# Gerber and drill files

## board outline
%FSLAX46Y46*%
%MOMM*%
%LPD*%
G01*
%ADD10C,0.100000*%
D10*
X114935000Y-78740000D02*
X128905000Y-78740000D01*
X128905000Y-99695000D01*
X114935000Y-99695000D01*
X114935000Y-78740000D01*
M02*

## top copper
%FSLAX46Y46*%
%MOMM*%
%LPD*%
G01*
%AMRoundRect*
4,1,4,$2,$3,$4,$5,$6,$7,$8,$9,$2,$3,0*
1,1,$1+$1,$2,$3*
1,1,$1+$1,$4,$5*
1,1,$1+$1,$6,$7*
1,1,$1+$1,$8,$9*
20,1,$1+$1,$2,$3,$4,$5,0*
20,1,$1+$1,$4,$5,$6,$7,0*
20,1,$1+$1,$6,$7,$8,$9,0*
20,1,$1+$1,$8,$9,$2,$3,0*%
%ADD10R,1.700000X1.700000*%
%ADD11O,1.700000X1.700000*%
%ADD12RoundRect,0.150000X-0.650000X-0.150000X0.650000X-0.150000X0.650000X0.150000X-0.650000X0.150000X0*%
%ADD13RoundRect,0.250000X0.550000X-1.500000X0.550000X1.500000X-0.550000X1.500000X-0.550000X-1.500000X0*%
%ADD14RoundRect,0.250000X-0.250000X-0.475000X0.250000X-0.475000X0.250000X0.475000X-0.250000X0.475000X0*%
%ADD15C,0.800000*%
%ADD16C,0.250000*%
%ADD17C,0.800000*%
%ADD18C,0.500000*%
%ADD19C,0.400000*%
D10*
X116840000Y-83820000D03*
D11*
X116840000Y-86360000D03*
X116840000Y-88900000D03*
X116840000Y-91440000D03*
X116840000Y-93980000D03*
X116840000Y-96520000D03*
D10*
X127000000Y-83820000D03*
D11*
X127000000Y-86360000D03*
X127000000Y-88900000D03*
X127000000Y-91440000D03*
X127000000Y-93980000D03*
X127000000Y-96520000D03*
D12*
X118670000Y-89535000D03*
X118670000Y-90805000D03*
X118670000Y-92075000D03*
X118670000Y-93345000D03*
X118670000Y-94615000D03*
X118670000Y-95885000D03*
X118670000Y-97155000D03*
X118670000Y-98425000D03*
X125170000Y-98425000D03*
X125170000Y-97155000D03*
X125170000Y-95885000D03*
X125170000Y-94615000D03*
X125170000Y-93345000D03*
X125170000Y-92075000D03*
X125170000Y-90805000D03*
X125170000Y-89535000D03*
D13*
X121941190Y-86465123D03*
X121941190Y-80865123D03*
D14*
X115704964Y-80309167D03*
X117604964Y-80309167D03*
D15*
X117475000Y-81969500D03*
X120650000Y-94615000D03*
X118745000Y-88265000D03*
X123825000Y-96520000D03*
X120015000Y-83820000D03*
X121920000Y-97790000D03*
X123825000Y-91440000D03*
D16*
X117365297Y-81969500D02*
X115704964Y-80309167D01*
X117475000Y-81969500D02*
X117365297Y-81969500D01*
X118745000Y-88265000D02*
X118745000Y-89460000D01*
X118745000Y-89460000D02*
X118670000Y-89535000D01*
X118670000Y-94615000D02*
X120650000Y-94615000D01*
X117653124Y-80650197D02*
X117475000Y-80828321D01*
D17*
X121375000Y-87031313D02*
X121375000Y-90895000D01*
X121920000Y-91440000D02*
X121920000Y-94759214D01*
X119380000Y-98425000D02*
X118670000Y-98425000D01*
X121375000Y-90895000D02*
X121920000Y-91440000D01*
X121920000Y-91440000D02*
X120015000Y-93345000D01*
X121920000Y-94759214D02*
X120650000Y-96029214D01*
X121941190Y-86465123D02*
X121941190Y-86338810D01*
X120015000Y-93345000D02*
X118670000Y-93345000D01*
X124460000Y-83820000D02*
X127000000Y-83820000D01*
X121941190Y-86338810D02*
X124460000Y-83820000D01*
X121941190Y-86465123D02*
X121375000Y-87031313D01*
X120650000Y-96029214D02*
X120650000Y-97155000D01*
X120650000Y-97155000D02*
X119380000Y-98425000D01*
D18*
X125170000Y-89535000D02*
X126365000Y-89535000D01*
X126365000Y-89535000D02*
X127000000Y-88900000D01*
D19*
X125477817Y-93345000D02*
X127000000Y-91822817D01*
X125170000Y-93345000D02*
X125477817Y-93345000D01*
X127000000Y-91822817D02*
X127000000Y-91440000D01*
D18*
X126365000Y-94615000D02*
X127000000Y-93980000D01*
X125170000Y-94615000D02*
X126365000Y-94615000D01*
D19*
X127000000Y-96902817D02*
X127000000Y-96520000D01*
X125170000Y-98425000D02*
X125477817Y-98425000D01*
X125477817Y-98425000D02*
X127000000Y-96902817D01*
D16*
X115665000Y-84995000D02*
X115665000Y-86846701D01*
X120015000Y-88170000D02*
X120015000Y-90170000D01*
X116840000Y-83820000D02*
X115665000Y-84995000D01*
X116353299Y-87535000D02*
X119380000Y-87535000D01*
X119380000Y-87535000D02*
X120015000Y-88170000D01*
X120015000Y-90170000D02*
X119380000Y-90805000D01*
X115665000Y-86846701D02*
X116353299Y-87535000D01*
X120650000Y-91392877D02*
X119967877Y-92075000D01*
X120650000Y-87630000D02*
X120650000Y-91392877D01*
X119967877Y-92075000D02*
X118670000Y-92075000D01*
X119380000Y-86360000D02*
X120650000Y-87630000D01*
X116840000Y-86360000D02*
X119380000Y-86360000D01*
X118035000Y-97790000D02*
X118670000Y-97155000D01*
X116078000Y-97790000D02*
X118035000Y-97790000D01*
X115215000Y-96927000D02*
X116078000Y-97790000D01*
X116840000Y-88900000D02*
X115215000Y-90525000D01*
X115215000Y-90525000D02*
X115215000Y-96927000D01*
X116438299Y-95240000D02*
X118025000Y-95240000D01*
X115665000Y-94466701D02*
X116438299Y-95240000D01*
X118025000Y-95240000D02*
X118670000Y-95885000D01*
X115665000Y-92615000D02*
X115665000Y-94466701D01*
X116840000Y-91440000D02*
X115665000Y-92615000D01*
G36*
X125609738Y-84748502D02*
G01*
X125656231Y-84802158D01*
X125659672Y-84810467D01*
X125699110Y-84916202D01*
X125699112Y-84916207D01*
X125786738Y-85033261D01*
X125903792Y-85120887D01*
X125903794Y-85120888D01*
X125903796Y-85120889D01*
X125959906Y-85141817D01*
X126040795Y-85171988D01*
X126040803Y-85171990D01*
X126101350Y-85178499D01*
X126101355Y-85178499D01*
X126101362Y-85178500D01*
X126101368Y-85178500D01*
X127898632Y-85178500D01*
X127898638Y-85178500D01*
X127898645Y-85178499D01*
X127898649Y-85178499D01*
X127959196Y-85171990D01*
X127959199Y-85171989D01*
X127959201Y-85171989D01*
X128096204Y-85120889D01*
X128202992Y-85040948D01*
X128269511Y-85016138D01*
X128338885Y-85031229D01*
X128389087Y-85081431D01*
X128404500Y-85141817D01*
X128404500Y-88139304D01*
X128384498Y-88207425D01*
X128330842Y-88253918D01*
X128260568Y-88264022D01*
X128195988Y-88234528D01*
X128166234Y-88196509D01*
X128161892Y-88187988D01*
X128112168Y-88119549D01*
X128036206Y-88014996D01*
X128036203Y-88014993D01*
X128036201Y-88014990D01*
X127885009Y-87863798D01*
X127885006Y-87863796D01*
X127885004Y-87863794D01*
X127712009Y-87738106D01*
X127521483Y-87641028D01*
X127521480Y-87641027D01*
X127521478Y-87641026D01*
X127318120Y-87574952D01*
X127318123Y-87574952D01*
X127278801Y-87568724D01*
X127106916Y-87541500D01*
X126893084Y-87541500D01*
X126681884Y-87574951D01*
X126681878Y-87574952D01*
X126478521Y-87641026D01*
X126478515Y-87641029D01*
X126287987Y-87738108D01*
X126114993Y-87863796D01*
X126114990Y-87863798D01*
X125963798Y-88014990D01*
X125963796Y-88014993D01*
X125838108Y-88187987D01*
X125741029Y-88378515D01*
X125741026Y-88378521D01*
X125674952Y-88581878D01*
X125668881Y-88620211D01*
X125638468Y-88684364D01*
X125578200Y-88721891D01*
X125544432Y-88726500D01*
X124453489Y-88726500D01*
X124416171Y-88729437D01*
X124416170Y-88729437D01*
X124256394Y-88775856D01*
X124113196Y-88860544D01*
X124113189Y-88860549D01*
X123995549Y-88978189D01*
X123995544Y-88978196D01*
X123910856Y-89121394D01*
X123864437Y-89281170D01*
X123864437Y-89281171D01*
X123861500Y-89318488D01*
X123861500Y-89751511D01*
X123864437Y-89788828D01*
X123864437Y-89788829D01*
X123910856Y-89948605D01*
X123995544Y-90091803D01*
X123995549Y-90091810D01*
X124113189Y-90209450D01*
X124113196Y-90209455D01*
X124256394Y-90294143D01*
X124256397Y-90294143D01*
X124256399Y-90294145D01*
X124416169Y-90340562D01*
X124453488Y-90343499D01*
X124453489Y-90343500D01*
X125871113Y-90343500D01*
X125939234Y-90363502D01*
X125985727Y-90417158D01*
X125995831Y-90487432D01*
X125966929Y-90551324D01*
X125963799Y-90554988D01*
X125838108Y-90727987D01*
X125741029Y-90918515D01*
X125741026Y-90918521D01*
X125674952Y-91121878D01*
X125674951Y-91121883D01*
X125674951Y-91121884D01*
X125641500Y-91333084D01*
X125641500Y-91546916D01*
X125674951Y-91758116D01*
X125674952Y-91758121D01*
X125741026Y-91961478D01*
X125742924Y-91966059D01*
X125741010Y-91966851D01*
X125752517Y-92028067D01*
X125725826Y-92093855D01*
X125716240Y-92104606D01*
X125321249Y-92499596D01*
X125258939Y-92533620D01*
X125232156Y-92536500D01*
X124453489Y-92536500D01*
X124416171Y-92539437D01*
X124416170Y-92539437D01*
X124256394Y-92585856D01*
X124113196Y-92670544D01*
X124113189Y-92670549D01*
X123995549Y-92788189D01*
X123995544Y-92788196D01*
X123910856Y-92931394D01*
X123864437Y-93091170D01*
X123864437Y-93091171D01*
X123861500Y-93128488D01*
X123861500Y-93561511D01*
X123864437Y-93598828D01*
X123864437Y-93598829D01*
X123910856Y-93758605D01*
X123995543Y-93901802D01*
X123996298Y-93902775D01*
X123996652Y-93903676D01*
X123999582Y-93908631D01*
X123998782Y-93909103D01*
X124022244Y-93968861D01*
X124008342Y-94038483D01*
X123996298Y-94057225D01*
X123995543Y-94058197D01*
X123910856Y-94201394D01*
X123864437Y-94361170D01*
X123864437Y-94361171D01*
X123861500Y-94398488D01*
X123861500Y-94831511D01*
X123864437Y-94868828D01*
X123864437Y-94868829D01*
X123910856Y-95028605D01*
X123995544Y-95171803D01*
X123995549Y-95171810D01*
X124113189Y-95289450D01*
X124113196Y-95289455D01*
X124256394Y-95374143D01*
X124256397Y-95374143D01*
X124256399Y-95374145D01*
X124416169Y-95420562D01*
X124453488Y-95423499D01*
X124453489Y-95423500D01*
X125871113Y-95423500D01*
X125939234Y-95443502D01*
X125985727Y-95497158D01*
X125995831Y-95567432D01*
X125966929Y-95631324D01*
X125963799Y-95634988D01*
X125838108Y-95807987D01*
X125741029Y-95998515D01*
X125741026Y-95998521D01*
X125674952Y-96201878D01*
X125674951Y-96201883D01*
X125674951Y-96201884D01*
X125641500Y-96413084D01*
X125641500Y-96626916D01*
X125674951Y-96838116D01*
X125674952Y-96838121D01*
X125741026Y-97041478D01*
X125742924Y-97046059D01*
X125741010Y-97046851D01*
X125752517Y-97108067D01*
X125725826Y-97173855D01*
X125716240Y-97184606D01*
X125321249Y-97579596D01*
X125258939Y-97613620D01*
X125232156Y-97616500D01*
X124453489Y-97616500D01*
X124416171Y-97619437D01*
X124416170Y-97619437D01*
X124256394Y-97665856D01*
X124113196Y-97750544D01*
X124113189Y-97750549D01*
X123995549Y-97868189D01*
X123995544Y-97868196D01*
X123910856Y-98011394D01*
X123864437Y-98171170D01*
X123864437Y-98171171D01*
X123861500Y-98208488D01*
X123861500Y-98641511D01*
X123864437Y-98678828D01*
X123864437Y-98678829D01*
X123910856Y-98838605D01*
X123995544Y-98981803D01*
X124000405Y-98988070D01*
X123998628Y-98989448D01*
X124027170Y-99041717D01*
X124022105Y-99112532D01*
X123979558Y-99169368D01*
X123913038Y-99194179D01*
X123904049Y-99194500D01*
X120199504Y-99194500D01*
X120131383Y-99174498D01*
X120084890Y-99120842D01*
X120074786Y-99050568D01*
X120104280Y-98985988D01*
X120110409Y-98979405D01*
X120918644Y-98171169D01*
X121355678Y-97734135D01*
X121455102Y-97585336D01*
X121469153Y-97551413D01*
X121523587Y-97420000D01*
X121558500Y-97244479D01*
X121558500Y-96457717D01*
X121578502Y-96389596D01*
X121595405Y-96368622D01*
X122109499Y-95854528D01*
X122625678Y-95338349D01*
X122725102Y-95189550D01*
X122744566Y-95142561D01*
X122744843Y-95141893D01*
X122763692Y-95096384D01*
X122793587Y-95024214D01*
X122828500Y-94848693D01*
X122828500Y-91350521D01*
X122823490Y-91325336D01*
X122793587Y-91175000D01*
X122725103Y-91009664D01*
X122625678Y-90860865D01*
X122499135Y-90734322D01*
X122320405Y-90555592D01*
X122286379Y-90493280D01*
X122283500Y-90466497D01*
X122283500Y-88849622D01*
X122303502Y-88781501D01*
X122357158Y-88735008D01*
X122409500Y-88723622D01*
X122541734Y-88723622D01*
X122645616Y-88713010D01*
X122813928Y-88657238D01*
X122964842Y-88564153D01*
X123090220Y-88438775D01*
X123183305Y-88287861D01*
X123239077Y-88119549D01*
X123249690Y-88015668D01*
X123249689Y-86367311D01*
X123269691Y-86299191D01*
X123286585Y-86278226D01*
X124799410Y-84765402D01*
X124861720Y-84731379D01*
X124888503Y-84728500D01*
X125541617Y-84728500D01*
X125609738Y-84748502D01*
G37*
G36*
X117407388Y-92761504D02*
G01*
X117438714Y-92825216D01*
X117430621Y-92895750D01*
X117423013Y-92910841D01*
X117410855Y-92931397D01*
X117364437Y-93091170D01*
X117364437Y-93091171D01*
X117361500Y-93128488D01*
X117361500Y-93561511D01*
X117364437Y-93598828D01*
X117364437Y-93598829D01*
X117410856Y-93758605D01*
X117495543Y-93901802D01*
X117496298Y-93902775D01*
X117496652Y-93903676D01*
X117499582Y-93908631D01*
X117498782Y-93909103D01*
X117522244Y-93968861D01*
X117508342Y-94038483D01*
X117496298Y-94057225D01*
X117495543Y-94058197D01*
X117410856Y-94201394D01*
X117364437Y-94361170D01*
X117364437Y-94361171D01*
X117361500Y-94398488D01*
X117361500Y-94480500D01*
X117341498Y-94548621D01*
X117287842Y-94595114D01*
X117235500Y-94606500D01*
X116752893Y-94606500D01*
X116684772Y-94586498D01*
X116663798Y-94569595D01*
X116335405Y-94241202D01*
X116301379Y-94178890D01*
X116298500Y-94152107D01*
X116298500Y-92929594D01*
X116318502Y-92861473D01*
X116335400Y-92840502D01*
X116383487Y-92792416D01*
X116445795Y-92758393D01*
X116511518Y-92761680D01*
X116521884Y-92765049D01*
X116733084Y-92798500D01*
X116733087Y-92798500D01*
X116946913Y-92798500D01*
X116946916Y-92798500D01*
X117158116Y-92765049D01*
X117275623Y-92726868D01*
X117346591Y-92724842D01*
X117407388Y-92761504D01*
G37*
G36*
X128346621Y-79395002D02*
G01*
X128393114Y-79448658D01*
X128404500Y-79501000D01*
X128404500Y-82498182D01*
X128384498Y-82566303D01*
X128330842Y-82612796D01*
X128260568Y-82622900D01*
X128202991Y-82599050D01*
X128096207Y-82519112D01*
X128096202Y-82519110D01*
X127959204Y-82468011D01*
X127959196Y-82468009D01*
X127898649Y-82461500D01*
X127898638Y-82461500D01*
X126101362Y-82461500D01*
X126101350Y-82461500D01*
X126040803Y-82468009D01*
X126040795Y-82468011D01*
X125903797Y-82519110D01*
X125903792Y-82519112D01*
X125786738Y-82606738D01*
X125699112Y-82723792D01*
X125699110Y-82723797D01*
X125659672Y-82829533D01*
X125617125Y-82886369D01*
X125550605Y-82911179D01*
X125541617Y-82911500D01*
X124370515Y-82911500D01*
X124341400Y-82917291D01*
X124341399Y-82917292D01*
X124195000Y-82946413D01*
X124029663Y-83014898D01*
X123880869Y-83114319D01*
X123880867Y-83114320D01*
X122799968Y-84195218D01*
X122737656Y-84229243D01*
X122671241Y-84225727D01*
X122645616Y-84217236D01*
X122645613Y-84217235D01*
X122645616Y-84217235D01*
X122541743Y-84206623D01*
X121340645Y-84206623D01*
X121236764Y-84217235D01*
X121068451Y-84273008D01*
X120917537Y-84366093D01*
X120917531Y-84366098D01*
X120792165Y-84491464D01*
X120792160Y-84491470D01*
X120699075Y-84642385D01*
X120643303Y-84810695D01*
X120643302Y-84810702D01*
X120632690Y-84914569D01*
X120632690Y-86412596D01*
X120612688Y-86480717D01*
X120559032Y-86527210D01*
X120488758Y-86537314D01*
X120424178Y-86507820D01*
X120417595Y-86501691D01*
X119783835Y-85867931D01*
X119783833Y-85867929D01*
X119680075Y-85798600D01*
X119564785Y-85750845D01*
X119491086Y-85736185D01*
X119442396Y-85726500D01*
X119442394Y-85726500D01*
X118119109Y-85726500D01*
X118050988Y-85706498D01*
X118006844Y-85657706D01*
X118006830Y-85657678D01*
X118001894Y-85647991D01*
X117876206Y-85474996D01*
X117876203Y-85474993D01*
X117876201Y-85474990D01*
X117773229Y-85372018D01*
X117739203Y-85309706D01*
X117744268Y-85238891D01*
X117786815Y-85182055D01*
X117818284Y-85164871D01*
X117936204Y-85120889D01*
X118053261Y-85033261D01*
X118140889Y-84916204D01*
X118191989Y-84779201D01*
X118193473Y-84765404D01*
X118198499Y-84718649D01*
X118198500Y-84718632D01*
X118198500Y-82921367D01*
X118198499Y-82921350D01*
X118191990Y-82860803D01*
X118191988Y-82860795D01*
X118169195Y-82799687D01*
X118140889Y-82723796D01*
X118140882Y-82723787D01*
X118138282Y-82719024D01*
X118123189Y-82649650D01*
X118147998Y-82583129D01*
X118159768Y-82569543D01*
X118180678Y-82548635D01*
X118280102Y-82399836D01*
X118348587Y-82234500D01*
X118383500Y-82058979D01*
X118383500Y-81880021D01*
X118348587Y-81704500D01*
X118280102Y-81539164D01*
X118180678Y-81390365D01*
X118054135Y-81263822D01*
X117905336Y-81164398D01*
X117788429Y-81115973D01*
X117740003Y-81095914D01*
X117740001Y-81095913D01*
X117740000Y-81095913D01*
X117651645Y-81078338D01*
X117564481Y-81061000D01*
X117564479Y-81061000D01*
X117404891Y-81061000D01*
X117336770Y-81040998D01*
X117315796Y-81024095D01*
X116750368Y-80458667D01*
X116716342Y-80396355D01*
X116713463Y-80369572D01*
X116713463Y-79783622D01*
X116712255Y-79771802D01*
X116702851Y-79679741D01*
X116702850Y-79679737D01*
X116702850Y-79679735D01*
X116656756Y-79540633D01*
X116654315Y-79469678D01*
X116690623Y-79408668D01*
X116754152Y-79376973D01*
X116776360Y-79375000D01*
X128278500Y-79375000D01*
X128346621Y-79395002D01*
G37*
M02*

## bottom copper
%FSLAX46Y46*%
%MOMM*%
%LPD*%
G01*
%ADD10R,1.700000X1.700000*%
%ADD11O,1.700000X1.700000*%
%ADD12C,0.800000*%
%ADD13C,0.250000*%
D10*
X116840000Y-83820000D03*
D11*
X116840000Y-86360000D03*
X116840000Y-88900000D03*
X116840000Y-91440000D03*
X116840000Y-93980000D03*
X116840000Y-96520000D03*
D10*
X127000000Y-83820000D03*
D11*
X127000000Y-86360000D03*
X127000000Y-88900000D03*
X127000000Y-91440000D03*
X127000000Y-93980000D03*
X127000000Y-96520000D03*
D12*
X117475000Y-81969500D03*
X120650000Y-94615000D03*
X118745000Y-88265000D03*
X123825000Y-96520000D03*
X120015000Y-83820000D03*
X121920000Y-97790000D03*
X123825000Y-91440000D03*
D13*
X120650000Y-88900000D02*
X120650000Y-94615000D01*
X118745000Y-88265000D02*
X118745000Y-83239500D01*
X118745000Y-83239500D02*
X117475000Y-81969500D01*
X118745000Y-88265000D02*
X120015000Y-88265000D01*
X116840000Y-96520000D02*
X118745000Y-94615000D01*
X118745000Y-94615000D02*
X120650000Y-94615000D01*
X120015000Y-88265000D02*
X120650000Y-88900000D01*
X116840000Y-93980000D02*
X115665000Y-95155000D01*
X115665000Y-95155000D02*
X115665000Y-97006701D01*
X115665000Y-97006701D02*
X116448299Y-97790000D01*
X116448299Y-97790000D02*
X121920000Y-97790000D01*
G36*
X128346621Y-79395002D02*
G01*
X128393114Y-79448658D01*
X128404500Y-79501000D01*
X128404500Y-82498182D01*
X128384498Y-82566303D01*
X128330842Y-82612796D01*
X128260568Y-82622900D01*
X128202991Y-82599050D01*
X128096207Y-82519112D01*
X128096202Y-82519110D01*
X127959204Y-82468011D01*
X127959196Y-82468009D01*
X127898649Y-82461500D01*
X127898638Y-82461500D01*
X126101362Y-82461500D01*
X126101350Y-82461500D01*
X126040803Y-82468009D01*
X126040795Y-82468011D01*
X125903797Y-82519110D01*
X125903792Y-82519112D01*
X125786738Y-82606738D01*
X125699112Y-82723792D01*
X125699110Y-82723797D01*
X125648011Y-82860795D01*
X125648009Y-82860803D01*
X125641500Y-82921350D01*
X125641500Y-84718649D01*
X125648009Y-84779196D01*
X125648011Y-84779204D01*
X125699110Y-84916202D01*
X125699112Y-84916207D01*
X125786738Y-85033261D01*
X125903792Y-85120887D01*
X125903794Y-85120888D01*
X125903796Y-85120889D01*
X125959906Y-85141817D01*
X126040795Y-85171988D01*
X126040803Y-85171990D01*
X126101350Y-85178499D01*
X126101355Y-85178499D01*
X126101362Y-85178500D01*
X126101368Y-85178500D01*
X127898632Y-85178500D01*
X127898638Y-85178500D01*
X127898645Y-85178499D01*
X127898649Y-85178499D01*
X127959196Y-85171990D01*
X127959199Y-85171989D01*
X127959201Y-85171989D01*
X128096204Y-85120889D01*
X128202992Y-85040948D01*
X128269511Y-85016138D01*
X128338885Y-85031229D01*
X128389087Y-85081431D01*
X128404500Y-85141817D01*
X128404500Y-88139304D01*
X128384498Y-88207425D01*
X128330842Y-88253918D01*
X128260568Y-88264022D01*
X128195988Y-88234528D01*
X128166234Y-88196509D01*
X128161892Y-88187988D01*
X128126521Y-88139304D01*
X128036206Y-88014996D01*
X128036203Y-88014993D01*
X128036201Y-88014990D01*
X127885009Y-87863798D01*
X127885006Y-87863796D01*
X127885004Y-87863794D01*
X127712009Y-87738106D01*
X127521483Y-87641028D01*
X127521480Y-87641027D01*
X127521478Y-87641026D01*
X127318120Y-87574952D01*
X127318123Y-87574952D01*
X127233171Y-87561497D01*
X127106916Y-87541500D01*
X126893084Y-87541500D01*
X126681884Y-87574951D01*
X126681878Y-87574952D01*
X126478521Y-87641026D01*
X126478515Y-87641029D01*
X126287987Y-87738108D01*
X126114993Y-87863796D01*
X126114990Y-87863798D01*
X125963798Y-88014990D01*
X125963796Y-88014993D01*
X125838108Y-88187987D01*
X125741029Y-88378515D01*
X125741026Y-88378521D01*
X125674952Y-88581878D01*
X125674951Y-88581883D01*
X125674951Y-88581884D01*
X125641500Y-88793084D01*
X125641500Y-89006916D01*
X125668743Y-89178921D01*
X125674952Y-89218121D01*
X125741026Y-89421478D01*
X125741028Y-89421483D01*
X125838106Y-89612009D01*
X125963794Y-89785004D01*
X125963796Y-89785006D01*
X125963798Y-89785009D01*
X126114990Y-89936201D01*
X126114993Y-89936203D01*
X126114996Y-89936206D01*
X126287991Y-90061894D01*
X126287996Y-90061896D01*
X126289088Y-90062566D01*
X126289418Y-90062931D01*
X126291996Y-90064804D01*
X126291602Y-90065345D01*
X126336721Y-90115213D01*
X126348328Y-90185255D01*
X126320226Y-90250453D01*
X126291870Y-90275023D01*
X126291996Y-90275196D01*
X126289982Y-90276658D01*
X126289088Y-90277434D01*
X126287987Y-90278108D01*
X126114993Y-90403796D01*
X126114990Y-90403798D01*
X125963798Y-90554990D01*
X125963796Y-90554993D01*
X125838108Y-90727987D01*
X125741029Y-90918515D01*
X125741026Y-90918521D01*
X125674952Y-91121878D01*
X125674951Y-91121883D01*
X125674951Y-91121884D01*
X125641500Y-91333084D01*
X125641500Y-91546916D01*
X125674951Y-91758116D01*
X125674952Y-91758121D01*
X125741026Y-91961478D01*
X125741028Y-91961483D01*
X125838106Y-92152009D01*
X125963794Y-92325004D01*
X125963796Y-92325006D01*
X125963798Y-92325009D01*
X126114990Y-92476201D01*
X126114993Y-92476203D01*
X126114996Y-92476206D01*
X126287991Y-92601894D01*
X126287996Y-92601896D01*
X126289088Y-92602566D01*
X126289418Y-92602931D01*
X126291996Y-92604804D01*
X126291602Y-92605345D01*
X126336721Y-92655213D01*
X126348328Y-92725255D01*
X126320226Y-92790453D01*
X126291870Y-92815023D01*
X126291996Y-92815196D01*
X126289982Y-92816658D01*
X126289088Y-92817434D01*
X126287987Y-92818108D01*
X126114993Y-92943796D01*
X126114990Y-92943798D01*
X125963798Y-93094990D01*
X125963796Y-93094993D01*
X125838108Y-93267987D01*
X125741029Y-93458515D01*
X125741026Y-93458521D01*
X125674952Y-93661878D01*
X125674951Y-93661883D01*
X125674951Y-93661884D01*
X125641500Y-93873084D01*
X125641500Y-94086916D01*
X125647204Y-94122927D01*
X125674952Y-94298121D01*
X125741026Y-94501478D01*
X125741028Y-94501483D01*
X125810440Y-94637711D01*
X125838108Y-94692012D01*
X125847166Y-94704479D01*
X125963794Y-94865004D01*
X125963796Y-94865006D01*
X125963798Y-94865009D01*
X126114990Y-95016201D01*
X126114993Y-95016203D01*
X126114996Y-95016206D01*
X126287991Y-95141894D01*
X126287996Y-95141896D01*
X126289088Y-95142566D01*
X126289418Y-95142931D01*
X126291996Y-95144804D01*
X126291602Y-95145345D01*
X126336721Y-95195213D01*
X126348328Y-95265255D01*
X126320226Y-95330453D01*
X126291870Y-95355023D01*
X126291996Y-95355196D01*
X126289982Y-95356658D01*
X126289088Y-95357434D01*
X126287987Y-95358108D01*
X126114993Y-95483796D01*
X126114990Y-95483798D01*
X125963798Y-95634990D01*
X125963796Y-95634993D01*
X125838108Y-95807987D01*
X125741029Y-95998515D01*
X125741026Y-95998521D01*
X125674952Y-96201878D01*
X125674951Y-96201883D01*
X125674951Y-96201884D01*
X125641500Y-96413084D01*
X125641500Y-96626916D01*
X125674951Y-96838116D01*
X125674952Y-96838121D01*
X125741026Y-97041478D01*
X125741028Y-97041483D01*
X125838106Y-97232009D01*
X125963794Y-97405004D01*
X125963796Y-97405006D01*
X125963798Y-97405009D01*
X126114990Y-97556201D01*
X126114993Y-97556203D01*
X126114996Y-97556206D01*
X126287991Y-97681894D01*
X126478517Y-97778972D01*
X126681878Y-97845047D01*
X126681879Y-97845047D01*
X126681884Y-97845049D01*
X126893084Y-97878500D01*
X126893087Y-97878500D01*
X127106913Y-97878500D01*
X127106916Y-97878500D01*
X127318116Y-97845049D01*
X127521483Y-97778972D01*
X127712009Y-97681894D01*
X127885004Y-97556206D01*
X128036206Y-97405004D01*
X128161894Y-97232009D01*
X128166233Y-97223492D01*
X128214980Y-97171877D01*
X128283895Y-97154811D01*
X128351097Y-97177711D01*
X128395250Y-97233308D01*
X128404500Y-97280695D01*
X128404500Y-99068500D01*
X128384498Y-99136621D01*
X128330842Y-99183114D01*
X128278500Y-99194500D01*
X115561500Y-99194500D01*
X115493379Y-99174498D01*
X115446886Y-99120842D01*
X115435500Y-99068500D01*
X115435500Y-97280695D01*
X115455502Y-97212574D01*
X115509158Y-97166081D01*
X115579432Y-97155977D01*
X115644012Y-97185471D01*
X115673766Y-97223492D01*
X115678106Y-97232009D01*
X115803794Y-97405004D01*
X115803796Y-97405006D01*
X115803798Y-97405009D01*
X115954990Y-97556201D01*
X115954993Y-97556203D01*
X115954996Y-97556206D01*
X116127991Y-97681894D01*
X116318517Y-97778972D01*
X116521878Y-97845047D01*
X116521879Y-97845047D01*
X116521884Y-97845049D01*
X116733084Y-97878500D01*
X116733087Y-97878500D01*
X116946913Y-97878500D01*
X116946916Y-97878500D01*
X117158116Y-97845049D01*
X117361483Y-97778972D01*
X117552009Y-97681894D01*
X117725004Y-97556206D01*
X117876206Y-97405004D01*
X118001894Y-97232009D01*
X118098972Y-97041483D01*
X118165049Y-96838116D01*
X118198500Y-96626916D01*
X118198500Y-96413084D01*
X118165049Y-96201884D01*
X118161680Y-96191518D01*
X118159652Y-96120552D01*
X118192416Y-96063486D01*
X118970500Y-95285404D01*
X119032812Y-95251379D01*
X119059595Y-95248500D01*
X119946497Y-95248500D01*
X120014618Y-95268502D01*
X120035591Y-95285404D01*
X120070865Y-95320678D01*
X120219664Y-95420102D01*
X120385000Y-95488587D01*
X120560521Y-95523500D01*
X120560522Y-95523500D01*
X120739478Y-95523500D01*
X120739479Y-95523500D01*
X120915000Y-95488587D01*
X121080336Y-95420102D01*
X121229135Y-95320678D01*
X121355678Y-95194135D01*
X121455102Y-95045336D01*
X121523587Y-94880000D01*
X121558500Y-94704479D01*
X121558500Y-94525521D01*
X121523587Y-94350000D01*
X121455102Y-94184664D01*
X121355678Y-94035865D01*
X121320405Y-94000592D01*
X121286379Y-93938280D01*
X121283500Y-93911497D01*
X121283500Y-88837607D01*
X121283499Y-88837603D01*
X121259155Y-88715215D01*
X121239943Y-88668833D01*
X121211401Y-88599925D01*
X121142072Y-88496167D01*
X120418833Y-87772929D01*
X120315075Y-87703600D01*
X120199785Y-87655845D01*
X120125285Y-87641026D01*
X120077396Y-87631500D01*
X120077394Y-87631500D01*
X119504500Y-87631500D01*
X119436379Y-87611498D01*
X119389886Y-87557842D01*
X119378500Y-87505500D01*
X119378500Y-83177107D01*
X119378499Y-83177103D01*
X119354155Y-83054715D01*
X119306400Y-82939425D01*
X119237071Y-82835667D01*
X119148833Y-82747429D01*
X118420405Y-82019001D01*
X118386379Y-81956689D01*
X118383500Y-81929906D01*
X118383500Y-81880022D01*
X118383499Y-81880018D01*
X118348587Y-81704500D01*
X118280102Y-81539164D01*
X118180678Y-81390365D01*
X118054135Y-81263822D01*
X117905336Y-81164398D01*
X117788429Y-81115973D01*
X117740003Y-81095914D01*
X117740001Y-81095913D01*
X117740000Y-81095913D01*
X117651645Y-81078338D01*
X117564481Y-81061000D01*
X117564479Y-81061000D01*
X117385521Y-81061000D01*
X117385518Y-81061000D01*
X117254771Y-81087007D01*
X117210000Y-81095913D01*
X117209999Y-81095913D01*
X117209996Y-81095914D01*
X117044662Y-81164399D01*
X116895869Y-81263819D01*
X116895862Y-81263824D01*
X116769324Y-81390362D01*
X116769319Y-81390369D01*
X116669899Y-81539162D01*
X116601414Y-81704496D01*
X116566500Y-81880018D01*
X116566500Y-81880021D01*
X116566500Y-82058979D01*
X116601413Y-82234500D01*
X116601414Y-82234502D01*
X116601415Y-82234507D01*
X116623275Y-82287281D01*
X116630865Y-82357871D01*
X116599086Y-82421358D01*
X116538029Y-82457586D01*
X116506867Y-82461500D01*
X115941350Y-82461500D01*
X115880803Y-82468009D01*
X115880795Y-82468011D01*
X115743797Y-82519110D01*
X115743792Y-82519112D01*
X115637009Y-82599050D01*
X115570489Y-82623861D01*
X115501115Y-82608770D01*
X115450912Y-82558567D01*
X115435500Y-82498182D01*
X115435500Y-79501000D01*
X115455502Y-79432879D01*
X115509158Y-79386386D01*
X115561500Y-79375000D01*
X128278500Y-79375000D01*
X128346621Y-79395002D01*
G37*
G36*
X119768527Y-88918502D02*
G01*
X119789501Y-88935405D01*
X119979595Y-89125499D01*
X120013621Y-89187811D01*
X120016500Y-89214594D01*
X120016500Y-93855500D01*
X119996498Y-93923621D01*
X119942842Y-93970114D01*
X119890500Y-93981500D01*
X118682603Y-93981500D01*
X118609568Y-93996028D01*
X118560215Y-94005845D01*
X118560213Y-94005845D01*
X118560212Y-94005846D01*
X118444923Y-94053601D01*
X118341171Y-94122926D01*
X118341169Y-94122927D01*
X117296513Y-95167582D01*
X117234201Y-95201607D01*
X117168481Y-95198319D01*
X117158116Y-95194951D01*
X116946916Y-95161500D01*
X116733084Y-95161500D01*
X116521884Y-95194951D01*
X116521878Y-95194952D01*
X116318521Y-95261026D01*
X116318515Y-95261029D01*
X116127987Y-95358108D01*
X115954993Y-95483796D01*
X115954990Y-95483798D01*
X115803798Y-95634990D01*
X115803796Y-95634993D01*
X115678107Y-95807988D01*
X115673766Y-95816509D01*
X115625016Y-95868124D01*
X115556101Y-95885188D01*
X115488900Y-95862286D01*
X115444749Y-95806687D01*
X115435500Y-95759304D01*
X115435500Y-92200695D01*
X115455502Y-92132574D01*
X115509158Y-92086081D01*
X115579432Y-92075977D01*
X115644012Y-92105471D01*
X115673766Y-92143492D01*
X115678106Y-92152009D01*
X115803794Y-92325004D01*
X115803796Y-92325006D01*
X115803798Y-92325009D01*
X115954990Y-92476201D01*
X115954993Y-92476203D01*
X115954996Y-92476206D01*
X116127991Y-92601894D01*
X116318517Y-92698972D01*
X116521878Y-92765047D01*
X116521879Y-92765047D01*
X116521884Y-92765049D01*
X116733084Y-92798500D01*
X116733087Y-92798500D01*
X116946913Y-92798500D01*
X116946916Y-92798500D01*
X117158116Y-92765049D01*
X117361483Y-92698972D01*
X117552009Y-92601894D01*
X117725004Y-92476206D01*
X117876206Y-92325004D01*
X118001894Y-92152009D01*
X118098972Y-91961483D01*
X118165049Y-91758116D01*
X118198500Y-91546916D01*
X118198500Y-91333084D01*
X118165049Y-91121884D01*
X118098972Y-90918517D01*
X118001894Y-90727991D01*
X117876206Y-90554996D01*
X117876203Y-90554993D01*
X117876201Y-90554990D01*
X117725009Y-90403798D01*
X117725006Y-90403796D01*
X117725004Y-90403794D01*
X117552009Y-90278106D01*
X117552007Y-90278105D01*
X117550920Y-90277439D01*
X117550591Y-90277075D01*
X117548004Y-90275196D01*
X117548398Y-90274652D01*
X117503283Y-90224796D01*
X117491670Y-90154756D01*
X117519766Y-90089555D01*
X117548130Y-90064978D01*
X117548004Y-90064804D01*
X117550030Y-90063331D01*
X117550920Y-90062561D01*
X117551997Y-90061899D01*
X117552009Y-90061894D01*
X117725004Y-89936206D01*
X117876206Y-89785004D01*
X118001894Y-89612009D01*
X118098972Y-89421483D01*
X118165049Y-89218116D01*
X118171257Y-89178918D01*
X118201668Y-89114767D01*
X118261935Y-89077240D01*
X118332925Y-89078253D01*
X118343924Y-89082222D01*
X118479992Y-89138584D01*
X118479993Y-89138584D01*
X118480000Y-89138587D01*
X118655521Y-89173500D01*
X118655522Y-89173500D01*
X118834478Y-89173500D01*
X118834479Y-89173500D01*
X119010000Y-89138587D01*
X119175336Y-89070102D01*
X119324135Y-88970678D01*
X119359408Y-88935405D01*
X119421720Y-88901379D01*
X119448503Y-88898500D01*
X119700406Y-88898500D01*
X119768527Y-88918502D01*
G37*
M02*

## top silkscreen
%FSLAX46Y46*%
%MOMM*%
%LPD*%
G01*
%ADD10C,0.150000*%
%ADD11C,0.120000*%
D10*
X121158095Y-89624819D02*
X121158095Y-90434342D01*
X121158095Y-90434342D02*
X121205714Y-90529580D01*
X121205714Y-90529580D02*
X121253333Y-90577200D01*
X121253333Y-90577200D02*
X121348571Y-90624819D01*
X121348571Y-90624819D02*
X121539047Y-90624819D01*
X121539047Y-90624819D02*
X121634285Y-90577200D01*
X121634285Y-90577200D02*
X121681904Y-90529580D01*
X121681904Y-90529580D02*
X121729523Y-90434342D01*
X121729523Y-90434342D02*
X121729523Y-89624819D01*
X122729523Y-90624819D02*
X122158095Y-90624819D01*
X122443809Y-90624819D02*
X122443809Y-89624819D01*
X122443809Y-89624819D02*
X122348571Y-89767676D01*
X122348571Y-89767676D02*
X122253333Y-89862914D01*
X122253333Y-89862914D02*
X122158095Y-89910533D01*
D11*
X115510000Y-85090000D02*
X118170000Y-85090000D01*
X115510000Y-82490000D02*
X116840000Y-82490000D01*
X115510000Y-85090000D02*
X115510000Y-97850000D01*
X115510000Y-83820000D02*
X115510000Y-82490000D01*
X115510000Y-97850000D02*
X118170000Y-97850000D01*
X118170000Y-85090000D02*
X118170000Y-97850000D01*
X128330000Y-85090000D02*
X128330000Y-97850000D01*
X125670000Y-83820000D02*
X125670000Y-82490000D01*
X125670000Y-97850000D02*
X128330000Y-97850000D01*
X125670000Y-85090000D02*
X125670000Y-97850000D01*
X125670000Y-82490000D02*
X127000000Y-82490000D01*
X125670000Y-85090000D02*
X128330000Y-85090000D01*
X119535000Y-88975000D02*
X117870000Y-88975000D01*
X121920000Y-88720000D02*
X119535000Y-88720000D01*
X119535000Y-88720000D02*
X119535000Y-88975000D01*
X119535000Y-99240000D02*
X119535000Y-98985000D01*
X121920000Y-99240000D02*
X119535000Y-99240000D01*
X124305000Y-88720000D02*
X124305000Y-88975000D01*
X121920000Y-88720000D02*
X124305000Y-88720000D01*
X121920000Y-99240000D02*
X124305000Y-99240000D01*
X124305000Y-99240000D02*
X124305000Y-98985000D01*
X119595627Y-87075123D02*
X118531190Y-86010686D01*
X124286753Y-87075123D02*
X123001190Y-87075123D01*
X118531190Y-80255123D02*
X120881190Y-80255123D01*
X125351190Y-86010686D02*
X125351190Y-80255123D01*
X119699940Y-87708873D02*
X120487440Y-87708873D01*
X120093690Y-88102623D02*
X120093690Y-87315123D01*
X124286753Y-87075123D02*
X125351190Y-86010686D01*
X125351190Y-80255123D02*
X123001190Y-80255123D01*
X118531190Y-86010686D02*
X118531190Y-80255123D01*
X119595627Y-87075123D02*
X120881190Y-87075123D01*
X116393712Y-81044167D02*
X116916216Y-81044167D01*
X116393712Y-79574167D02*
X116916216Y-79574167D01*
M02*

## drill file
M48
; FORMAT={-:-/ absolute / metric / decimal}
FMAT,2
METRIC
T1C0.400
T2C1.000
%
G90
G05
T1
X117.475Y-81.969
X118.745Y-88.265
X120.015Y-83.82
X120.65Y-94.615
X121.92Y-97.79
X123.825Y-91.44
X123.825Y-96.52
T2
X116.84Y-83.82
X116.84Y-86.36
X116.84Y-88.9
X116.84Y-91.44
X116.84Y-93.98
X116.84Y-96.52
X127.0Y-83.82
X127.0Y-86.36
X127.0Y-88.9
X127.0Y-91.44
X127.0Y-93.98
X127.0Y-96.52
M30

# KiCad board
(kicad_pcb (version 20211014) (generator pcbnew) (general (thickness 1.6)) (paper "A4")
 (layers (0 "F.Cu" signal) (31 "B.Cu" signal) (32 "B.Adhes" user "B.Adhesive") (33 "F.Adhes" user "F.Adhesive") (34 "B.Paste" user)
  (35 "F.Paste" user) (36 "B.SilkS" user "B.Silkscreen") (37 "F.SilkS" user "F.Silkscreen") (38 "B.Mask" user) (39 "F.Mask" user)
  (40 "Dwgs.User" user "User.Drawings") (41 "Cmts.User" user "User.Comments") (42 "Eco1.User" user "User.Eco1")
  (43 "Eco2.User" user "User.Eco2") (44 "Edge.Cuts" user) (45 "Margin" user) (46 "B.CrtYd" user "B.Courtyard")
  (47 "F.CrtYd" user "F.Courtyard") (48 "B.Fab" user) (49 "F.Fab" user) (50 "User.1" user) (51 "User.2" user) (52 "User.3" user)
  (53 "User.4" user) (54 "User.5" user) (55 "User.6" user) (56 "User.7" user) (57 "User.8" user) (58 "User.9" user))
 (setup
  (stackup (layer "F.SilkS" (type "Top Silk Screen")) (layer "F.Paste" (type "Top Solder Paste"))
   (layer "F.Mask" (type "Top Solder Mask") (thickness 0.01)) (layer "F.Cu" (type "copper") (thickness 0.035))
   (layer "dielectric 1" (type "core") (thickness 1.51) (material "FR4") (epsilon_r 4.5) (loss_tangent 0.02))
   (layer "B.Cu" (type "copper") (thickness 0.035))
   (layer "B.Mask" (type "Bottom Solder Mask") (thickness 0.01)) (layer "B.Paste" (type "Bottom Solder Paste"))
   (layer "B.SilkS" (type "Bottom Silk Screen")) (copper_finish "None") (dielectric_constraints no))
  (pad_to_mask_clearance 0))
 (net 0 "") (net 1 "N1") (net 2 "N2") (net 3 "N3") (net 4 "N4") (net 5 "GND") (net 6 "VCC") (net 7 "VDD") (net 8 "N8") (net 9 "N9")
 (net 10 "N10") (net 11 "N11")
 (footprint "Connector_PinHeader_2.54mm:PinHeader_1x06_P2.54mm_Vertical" (layer "F.Cu") (at 116.84 83.82)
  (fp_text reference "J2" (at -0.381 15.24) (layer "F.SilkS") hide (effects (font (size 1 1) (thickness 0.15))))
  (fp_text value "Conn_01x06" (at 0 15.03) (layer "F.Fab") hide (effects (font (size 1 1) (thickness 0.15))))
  (fp_line (start -1.33 1.27) (end 1.33 1.27) (layer "F.SilkS") (width 0.12))
  (fp_line (start -1.33 -1.33) (end 0 -1.33) (layer "F.SilkS") (width 0.12))
  (fp_line (start -1.33 1.27) (end -1.33 14.03) (layer "F.SilkS") (width 0.12))
  (fp_line (start -1.33 0) (end -1.33 -1.33) (layer "F.SilkS") (width 0.12))
  (fp_line (start -1.33 14.03) (end 1.33 14.03) (layer "F.SilkS") (width 0.12))
  (fp_line (start 1.33 1.27) (end 1.33 14.03) (layer "F.SilkS") (width 0.12))
  (pad "1" thru_hole rect (at 0 0) (size 1.7 1.7) (drill 1) (layers *.Cu *.Mask) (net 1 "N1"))
  (pad "2" thru_hole oval (at 0 2.54) (size 1.7 1.7) (drill 1) (layers *.Cu *.Mask) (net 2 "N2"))
  (pad "3" thru_hole oval (at 0 5.08) (size 1.7 1.7) (drill 1) (layers *.Cu *.Mask) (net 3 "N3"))
  (pad "4" thru_hole oval (at 0 7.62) (size 1.7 1.7) (drill 1) (layers *.Cu *.Mask) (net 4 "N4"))
  (pad "5" thru_hole oval (at 0 10.16) (size 1.7 1.7) (drill 1) (layers *.Cu *.Mask) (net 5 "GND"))
  (pad "6" thru_hole oval (at 0 12.7) (size 1.7 1.7) (drill 1) (layers *.Cu *.Mask) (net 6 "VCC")))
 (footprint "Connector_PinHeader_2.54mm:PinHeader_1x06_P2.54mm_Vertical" (layer "F.Cu") (at 127 83.82)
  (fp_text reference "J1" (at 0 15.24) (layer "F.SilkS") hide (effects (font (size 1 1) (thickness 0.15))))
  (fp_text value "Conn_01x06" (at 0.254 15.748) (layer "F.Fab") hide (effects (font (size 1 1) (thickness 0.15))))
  (fp_line (start 1.33 1.27) (end 1.33 14.03) (layer "F.SilkS") (width 0.12))
  (fp_line (start -1.33 0) (end -1.33 -1.33) (layer "F.SilkS") (width 0.12))
  (fp_line (start -1.33 14.03) (end 1.33 14.03) (layer "F.SilkS") (width 0.12))
  (fp_line (start -1.33 1.27) (end -1.33 14.03) (layer "F.SilkS") (width 0.12))
  (fp_line (start -1.33 -1.33) (end 0 -1.33) (layer "F.SilkS") (width 0.12))
  (fp_line (start -1.33 1.27) (end 1.33 1.27) (layer "F.SilkS") (width 0.12))
  (pad "1" thru_hole rect (at 0 0) (size 1.7 1.7) (drill 1) (layers *.Cu *.Mask) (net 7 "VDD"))
  (pad "2" thru_hole oval (at 0 2.54) (size 1.7 1.7) (drill 1) (layers *.Cu *.Mask) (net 5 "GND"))
  (pad "3" thru_hole oval (at 0 5.08) (size 1.7 1.7) (drill 1) (layers *.Cu *.Mask) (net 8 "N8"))
  (pad "4" thru_hole oval (at 0 7.62) (size 1.7 1.7) (drill 1) (layers *.Cu *.Mask) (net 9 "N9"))
  (pad "5" thru_hole oval (at 0 10.16) (size 1.7 1.7) (drill 1) (layers *.Cu *.Mask) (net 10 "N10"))
  (pad "6" thru_hole oval (at 0 12.7) (size 1.7 1.7) (drill 1) (layers *.Cu *.Mask) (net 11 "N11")))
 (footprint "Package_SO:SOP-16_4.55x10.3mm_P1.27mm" (layer "F.Cu") (at 121.92 93.98)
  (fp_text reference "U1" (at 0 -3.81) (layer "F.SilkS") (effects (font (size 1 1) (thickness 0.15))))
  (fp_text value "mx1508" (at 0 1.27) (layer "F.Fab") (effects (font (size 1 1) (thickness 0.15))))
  (fp_line (start -2.385 -5.005) (end -4.05 -5.005) (layer "F.SilkS") (width 0.12))
  (fp_line (start 0 -5.26) (end -2.385 -5.26) (layer "F.SilkS") (width 0.12))
  (fp_line (start -2.385 -5.26) (end -2.385 -5.005) (layer "F.SilkS") (width 0.12))
  (fp_line (start -2.385 5.26) (end -2.385 5.005) (layer "F.SilkS") (width 0.12))
  (fp_line (start 0 5.26) (end -2.385 5.26) (layer "F.SilkS") (width 0.12))
  (fp_line (start 2.385 -5.26) (end 2.385 -5.005) (layer "F.SilkS") (width 0.12))
  (fp_line (start 0 -5.26) (end 2.385 -5.26) (layer "F.SilkS") (width 0.12))
  (fp_line (start 0 5.26) (end 2.385 5.26) (layer "F.SilkS") (width 0.12))
  (fp_line (start 2.385 5.26) (end 2.385 5.005) (layer "F.SilkS") (width 0.12))
  (pad "1" smd roundrect (at -3.25 -4.445) (size 1.6 0.6) (layers "F.Cu" "F.Paste" "F.Mask") (roundrect_rratio 0.25) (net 6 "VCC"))
  (pad "2" smd roundrect (at -3.25 -3.175) (size 1.6 0.6) (layers "F.Cu" "F.Paste" "F.Mask") (roundrect_rratio 0.25) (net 1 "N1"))
  (pad "3" smd roundrect (at -3.25 -1.905) (size 1.6 0.6) (layers "F.Cu" "F.Paste" "F.Mask") (roundrect_rratio 0.25) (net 2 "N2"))
  (pad "4" smd roundrect (at -3.25 -0.635) (size 1.6 0.6) (layers "F.Cu" "F.Paste" "F.Mask") (roundrect_rratio 0.25) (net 7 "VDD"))
  (pad "5" smd roundrect (at -3.25 0.635) (size 1.6 0.6) (layers "F.Cu" "F.Paste" "F.Mask") (roundrect_rratio 0.25) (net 6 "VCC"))
  (pad "6" smd roundrect (at -3.25 1.905) (size 1.6 0.6) (layers "F.Cu" "F.Paste" "F.Mask") (roundrect_rratio 0.25) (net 4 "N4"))
  (pad "7" smd roundrect (at -3.25 3.175) (size 1.6 0.6) (layers "F.Cu" "F.Paste" "F.Mask") (roundrect_rratio 0.25) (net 3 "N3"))
  (pad "8" smd roundrect (at -3.25 4.445) (size 1.6 0.6) (layers "F.Cu" "F.Paste" "F.Mask") (roundrect_rratio 0.25) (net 7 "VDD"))
  (pad "9" smd roundrect (at 3.25 4.445) (size 1.6 0.6) (layers "F.Cu" "F.Paste" "F.Mask") (roundrect_rratio 0.25) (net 11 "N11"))
  (pad "10" smd roundrect (at 3.25 3.175) (size 1.6 0.6) (layers "F.Cu" "F.Paste" "F.Mask") (roundrect_rratio 0.25) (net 5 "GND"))
  (pad "11" smd roundrect (at 3.25 1.905) (size 1.6 0.6) (layers "F.Cu" "F.Paste" "F.Mask") (roundrect_rratio 0.25) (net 5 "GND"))
  (pad "12" smd roundrect (at 3.25 0.635) (size 1.6 0.6) (layers "F.Cu" "F.Paste" "F.Mask") (roundrect_rratio 0.25) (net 10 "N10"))
  (pad "13" smd roundrect (at 3.25 -0.635) (size 1.6 0.6) (layers "F.Cu" "F.Paste" "F.Mask") (roundrect_rratio 0.25) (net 9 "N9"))
  (pad "14" smd roundrect (at 3.25 -1.905) (size 1.6 0.6) (layers "F.Cu" "F.Paste" "F.Mask") (roundrect_rratio 0.25) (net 5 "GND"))
  (pad "15" smd roundrect (at 3.25 -3.175) (size 1.6 0.6) (layers "F.Cu" "F.Paste" "F.Mask") (roundrect_rratio 0.25) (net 5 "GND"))
  (pad "16" smd roundrect (at 3.25 -4.445) (size 1.6 0.6) (layers "F.Cu" "F.Paste" "F.Mask") (roundrect_rratio 0.25) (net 8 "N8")))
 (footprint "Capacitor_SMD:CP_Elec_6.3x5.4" (layer "F.Cu") (at 121.94119 83.665123 90)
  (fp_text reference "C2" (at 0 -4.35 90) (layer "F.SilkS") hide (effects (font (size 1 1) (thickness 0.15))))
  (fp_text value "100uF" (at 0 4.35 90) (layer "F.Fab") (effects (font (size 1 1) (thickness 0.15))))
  (fp_line (start -3.41 -2.345563) (end -2.345563 -3.41) (layer "F.SilkS") (width 0.12))
  (fp_line (start -3.41 2.345563) (end -3.41 1.06) (layer "F.SilkS") (width 0.12))
  (fp_line (start 3.41 -3.41) (end 3.41 -1.06) (layer "F.SilkS") (width 0.12))
  (fp_line (start -2.345563 3.41) (end 3.41 3.41) (layer "F.SilkS") (width 0.12))
  (fp_line (start -4.04375 -2.24125) (end -4.04375 -1.45375) (layer "F.SilkS") (width 0.12))
  (fp_line (start -4.4375 -1.8475) (end -3.65 -1.8475) (layer "F.SilkS") (width 0.12))
  (fp_line (start -3.41 2.345563) (end -2.345563 3.41) (layer "F.SilkS") (width 0.12))
  (fp_line (start 3.41 3.41) (end 3.41 1.06) (layer "F.SilkS") (width 0.12))
  (fp_line (start -2.345563 -3.41) (end 3.41 -3.41) (layer "F.SilkS") (width 0.12))
  (fp_line (start -3.41 -2.345563) (end -3.41 -1.06) (layer "F.SilkS") (width 0.12))
  (pad "1" smd roundrect (at -2.8 0 90) (size 3.5 1.6) (layers "F.Cu" "F.Paste" "F.Mask") (roundrect_rratio 0.15625) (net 7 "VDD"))
  (pad "2" smd roundrect (at 2.8 0 90) (size 3.5 1.6) (layers "F.Cu" "F.Paste" "F.Mask") (roundrect_rratio 0.15625) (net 5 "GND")))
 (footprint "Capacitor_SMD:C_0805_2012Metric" (layer "F.Cu") (at 116.654964 80.309167)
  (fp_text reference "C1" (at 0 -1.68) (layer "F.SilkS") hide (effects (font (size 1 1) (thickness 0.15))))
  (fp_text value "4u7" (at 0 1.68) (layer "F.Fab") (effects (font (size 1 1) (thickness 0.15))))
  (fp_line (start -0.261252 0.735) (end 0.261252 0.735) (layer "F.SilkS") (width 0.12))
  (fp_line (start -0.261252 -0.735) (end 0.261252 -0.735) (layer "F.SilkS") (width 0.12))
  (pad "1" smd roundrect (at -0.95 0) (size 1 1.45) (layers "F.Cu" "F.Paste" "F.Mask") (roundrect_rratio 0.25) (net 6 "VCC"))
  (pad "2" smd roundrect (at 0.95 0) (size 1 1.45) (layers "F.Cu" "F.Paste" "F.Mask") (roundrect_rratio 0.25) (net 5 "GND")))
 (gr_rect (start 128.905 78.74) (end 114.935 99.695) (layer "Edge.Cuts") (width 0.1) (fill none))
 (segment (start 117.365297 81.9695) (end 115.704964 80.309167) (width 0.25) (layer "F.Cu") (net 6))
 (segment (start 117.475 81.9695) (end 117.365297 81.9695) (width 0.25) (layer "F.Cu") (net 6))
 (segment (start 118.745 88.265) (end 118.745 89.46) (width 0.25) (layer "F.Cu") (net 6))
 (segment (start 118.745 89.46) (end 118.67 89.535) (width 0.25) (layer "F.Cu") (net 6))
 (segment (start 118.67 94.615) (end 120.65 94.615) (width 0.25) (layer "F.Cu") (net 6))
 (via (at 117.475 81.9695) (size 0.8) (drill 0.4) (layers "F.Cu" "B.Cu") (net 6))
 (via (at 120.65 94.615) (size 0.8) (drill 0.4) (layers "F.Cu" "B.Cu") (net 6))
 (via (at 118.745 88.265) (size 0.8) (drill 0.4) (layers "F.Cu" "B.Cu") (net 6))
 (segment (start 120.65 88.9) (end 120.65 94.615) (width 0.25) (layer "B.Cu") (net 6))
 (segment (start 118.745 88.265) (end 118.745 83.2395) (width 0.25) (layer "B.Cu") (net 6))
 (segment (start 118.745 83.2395) (end 117.475 81.9695) (width 0.25) (layer "B.Cu") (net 6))
 (segment (start 118.745 88.265) (end 120.015 88.265) (width 0.25) (layer "B.Cu") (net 6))
 (segment (start 116.84 96.52) (end 118.745 94.615) (width 0.25) (layer "B.Cu") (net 6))
 (segment (start 118.745 94.615) (end 120.65 94.615) (width 0.25) (layer "B.Cu") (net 6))
 (segment (start 120.015 88.265) (end 120.65 88.9) (width 0.25) (layer "B.Cu") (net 6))
 (segment (start 117.653124 80.650197) (end 117.475 80.828321) (width 0.25) (layer "F.Cu") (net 5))
 (via (at 123.825 96.52) (size 0.8) (drill 0.4) (layers "F.Cu" "B.Cu") (free) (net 5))
 (via (at 120.015 83.82) (size 0.8) (drill 0.4) (layers "F.Cu" "B.Cu") (free) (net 5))
 (via (at 121.92 97.79) (size 0.8) (drill 0.4) (layers "F.Cu" "B.Cu") (free) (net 5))
 (via (at 123.825 91.44) (size 0.8) (drill 0.4) (layers "F.Cu" "B.Cu") (free) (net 5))
 (segment (start 116.84 93.98) (end 115.665 95.155) (width 0.25) (layer "B.Cu") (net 5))
 (segment (start 115.665 95.155) (end 115.665 97.006701) (width 0.25) (layer "B.Cu") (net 5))
 (segment (start 115.665 97.006701) (end 116.448299 97.79) (width 0.25) (layer "B.Cu") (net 5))
 (segment (start 116.448299 97.79) (end 121.92 97.79) (width 0.25) (layer "B.Cu") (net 5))
 (segment (start 121.375 87.031313) (end 121.375 90.895) (width 0.8) (layer "F.Cu") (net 7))
 (segment (start 121.92 91.44) (end 121.92 94.759214) (width 0.8) (layer "F.Cu") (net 7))
 (segment (start 119.38 98.425) (end 118.67 98.425) (width 0.8) (layer "F.Cu") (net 7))
 (segment (start 121.375 90.895) (end 121.92 91.44) (width 0.8) (layer "F.Cu") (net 7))
 (segment (start 121.92 91.44) (end 120.015 93.345) (width 0.8) (layer "F.Cu") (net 7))
 (segment (start 121.92 94.759214) (end 120.65 96.029214) (width 0.8) (layer "F.Cu") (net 7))
 (segment (start 121.94119 86.465123) (end 121.94119 86.33881) (width 0.8) (layer "F.Cu") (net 7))
 (segment (start 120.015 93.345) (end 118.67 93.345) (width 0.8) (layer "F.Cu") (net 7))
 (segment (start 124.46 83.82) (end 127 83.82) (width 0.8) (layer "F.Cu") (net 7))
 (segment (start 121.94119 86.33881) (end 124.46 83.82) (width 0.8) (layer "F.Cu") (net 7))
 (segment (start 121.94119 86.465123) (end 121.375 87.031313) (width 0.8) (layer "F.Cu") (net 7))
 (segment (start 120.65 96.029214) (end 120.65 97.155) (width 0.8) (layer "F.Cu") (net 7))
 (segment (start 120.65 97.155) (end 119.38 98.425) (width 0.8) (layer "F.Cu") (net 7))
 (segment (start 125.17 89.535) (end 126.365 89.535) (width 0.5) (layer "F.Cu") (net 8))
 (segment (start 126.365 89.535) (end 127 88.9) (width 0.5) (layer "F.Cu") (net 8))
 (segment (start 125.477817 93.345) (end 127 91.822817) (width 0.4) (layer "F.Cu") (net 9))
 (segment (start 125.17 93.345) (end 125.477817 93.345) (width 0.4) (layer "F.Cu") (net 9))
 (segment (start 127 91.822817) (end 127 91.44) (width 0.4) (layer "F.Cu") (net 9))
 (segment (start 126.365 94.615) (end 127 93.98) (width 0.5) (layer "F.Cu") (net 10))
 (segment (start 125.17 94.615) (end 126.365 94.615) (width 0.5) (layer "F.Cu") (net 10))
 (segment (start 127 96.902817) (end 127 96.52) (width 0.4) (layer "F.Cu") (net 11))
 (segment (start 125.17 98.425) (end 125.477817 98.425) (width 0.4) (layer "F.Cu") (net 11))
 (segment (start 125.477817 98.425) (end 127 96.902817) (width 0.4) (layer "F.Cu") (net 11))
 (segment (start 115.665 84.995) (end 115.665 86.846701) (width 0.25) (layer "F.Cu") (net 1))
 (segment (start 120.015 88.17) (end 120.015 90.17) (width 0.25) (layer "F.Cu") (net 1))
 (segment (start 116.84 83.82) (end 115.665 84.995) (width 0.25) (layer "F.Cu") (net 1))
 (segment (start 116.353299 87.535) (end 119.38 87.535) (width 0.25) (layer "F.Cu") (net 1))
 (segment (start 119.38 87.535) (end 120.015 88.17) (width 0.25) (layer "F.Cu") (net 1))
 (segment (start 120.015 90.17) (end 119.38 90.805) (width 0.25) (layer "F.Cu") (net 1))
 (segment (start 115.665 86.846701) (end 116.353299 87.535) (width 0.25) (layer "F.Cu") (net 1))
 (segment (start 120.65 91.392877) (end 119.967877 92.075) (width 0.25) (layer "F.Cu") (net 2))
 (segment (start 120.65 87.63) (end 120.65 91.392877) (width 0.25) (layer "F.Cu") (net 2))
 (segment (start 119.967877 92.075) (end 118.67 92.075) (width 0.25) (layer "F.Cu") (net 2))
 (segment (start 119.38 86.36) (end 120.65 87.63) (width 0.25) (layer "F.Cu") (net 2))
 (segment (start 116.84 86.36) (end 119.38 86.36) (width 0.25) (layer "F.Cu") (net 2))
 (segment (start 118.035 97.79) (end 118.67 97.155) (width 0.25) (layer "F.Cu") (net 3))
 (segment (start 116.078 97.79) (end 118.035 97.79) (width 0.25) (layer "F.Cu") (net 3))
 (segment (start 115.215 96.927) (end 116.078 97.79) (width 0.25) (layer "F.Cu") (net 3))
 (segment (start 116.84 88.9) (end 115.215 90.525) (width 0.25) (layer "F.Cu") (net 3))
 (segment (start 115.215 90.525) (end 115.215 96.927) (width 0.25) (layer "F.Cu") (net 3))
 (segment (start 116.438299 95.24) (end 118.025 95.24) (width 0.25) (layer "F.Cu") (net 4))
 (segment (start 115.665 94.466701) (end 116.438299 95.24) (width 0.25) (layer "F.Cu") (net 4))
 (segment (start 118.025 95.24) (end 118.67 95.885) (width 0.25) (layer "F.Cu") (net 4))
 (segment (start 115.665 92.615) (end 115.665 94.466701) (width 0.25) (layer "F.Cu") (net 4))
 (segment (start 116.84 91.44) (end 115.665 92.615) (width 0.25) (layer "F.Cu") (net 4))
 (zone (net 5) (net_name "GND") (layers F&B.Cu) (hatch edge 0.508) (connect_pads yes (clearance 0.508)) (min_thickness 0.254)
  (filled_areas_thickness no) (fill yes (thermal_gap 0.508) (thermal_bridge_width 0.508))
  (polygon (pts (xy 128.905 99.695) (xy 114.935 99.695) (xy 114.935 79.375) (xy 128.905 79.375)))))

